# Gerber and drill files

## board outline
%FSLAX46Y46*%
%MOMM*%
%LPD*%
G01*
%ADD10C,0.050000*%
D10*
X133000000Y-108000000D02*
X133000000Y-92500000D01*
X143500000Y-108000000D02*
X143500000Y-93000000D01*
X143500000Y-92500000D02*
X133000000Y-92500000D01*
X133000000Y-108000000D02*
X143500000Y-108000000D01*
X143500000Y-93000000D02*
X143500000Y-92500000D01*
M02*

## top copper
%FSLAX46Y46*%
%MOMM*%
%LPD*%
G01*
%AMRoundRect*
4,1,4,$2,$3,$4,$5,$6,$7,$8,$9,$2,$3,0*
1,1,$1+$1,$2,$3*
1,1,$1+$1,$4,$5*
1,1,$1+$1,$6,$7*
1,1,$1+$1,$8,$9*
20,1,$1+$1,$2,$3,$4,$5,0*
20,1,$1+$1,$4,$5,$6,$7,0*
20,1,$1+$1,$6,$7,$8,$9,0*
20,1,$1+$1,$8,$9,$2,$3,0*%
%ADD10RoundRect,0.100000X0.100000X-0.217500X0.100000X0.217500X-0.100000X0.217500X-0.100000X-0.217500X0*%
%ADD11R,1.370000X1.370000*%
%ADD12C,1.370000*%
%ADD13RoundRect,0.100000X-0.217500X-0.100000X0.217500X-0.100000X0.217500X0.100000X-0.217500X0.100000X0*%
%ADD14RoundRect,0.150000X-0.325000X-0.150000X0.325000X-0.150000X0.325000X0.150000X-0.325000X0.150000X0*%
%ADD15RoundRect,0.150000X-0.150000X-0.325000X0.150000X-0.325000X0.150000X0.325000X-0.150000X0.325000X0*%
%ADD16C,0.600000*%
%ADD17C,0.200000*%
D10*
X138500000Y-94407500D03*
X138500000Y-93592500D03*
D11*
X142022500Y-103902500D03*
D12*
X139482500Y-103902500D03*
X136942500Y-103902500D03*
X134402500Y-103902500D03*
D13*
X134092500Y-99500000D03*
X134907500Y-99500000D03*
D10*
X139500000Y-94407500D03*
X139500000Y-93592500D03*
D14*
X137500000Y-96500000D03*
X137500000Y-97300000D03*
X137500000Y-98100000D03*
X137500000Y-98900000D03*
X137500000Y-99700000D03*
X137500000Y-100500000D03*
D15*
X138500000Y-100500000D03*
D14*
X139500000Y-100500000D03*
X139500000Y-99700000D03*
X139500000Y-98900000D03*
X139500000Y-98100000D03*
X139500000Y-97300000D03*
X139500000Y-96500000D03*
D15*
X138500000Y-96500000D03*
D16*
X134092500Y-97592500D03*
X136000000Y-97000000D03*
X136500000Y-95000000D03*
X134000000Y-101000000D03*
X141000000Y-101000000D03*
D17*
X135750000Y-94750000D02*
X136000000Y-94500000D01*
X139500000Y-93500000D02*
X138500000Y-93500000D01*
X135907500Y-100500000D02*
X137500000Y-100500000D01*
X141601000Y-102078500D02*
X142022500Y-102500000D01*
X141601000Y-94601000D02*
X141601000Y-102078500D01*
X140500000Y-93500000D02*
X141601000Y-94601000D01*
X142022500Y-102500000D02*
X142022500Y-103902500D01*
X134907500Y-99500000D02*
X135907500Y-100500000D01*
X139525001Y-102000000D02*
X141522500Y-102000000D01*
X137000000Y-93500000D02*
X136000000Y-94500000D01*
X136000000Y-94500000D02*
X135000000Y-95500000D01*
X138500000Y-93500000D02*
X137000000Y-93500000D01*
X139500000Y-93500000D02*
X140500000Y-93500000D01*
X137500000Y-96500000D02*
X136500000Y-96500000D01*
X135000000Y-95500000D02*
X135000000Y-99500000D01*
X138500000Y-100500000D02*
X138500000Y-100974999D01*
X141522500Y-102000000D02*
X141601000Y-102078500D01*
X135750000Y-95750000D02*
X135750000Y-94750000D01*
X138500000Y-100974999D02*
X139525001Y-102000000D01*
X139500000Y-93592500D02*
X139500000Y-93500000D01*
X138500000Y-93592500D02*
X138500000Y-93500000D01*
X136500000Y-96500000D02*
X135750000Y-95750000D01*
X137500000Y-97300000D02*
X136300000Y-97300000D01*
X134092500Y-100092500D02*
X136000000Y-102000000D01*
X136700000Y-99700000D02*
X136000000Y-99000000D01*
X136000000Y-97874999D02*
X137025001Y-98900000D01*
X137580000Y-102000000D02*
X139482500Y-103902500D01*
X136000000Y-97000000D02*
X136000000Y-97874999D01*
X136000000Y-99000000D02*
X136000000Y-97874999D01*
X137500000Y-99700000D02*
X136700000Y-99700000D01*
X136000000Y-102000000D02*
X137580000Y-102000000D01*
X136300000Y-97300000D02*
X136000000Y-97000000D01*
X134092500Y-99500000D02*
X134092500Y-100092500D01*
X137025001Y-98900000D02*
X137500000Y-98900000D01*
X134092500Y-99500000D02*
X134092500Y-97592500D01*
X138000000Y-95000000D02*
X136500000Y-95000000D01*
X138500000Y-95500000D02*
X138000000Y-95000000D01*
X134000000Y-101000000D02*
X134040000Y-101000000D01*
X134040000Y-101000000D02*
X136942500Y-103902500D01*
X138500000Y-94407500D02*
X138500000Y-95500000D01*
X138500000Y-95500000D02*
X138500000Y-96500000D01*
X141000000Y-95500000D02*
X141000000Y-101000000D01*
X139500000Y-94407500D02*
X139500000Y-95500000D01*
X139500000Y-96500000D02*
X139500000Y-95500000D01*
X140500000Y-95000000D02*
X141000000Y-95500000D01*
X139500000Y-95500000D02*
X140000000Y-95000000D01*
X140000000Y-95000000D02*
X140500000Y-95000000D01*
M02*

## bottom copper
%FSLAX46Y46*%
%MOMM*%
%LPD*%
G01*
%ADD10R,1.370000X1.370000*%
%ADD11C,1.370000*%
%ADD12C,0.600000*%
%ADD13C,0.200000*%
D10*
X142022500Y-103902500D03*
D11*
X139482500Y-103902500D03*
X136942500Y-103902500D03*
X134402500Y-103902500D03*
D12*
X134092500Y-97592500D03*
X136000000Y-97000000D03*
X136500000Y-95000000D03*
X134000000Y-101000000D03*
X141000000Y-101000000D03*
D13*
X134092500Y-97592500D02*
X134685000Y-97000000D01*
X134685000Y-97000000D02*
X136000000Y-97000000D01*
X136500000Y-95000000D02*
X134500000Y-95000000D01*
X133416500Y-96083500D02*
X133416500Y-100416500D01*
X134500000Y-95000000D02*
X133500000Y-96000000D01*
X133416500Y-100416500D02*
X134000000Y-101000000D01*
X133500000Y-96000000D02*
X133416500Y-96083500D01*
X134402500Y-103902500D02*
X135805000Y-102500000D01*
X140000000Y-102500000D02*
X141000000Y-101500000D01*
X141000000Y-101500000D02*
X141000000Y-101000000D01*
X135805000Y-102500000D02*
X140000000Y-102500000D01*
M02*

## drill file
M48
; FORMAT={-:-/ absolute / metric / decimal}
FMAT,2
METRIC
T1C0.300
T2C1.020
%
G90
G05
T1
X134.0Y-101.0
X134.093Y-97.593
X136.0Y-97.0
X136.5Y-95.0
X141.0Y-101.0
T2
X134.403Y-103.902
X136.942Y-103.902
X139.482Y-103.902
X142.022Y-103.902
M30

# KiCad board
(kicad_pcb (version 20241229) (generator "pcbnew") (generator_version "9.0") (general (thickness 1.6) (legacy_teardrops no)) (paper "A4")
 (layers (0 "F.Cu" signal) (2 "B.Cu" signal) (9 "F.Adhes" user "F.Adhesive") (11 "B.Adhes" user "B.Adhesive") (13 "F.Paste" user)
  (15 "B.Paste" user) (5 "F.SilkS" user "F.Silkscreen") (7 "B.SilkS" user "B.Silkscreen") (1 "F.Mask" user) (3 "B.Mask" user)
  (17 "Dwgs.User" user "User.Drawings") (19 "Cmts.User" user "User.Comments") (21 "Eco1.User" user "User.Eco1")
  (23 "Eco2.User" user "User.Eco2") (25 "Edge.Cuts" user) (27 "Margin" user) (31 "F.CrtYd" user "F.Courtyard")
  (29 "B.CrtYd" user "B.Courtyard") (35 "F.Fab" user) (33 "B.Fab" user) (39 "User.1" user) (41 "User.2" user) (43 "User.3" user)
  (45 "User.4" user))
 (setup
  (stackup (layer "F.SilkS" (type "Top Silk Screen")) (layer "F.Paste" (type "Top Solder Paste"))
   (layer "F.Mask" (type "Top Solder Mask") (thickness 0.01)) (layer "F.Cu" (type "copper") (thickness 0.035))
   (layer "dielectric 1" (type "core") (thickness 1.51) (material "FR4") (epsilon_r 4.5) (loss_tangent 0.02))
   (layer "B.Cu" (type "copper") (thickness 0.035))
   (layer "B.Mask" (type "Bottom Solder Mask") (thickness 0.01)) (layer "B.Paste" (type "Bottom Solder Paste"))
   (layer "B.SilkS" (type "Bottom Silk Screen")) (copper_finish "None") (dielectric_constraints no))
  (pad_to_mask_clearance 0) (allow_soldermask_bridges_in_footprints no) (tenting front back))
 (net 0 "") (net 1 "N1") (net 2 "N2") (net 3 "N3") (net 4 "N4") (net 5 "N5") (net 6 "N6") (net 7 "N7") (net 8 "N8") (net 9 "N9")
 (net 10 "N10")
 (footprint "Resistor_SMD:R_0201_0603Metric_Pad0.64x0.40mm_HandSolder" (layer "F.Cu") (at 138.5 94 90)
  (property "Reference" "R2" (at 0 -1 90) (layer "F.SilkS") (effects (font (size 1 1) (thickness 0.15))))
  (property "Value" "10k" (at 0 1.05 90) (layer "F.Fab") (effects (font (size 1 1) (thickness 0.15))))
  (pad "" smd roundrect (at -0.4325 0 90) (size 0.458 0.36) (layers "F.Paste") (roundrect_rratio 0.25))
  (pad "" smd roundrect (at 0.4325 0 90) (size 0.458 0.36) (layers "F.Paste") (roundrect_rratio 0.25))
  (pad "1" smd roundrect (at -0.4075 0 90) (size 0.635 0.4) (layers "F.Cu" "F.Mask") (roundrect_rratio 0.25) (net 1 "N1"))
  (pad "2" smd roundrect (at 0.4075 0 90) (size 0.635 0.4) (layers "F.Cu" "F.Mask") (roundrect_rratio 0.25) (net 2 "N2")))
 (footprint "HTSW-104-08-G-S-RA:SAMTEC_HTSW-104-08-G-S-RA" (layer "F.Cu") (at 138.2125 106.6725)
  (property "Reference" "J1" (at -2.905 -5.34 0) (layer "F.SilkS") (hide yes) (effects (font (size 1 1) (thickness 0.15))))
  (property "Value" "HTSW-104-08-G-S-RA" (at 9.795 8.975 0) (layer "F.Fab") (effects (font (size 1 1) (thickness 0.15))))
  (pad "01" thru_hole rect (at 3.81 -2.77) (size 1.37 1.37) (drill 1.02) (layers "*.Cu" "*.Mask") (remove_unused_layers no) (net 2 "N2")
   (solder_mask_margin 0.102))
  (pad "02" thru_hole circle (at 1.27 -2.77) (size 1.37 1.37) (drill 1.02) (layers "*.Cu" "*.Mask") (remove_unused_layers no) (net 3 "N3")
   (solder_mask_margin 0.102))
  (pad "03" thru_hole circle (at -1.27 -2.77) (size 1.37 1.37) (drill 1.02) (layers "*.Cu" "*.Mask") (remove_unused_layers no) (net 1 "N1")
   (solder_mask_margin 0.102))
  (pad "04" thru_hole circle (at -3.81 -2.77) (size 1.37 1.37) (drill 1.02) (layers "*.Cu" "*.Mask") (remove_unused_layers no) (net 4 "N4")
   (solder_mask_margin 0.102)))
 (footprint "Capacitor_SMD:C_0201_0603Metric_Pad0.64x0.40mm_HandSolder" (layer "F.Cu") (at 134.5 99.5)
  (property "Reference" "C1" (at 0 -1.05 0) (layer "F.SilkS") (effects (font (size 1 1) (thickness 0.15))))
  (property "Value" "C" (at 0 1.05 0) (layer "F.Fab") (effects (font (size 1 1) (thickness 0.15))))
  (pad "" smd roundrect (at -0.4325 0) (size 0.458 0.36) (layers "F.Paste") (roundrect_rratio 0.25))
  (pad "" smd roundrect (at 0.4325 0) (size 0.458 0.36) (layers "F.Paste") (roundrect_rratio 0.25))
  (pad "1" smd roundrect (at -0.4075 0) (size 0.635 0.4) (layers "F.Cu" "F.Mask") (roundrect_rratio 0.25) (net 3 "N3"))
  (pad "2" smd roundrect (at 0.4075 0) (size 0.635 0.4) (layers "F.Cu" "F.Mask") (roundrect_rratio 0.25) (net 2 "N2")))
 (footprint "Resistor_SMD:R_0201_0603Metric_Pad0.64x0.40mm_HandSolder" (layer "F.Cu") (at 139.5 94 90)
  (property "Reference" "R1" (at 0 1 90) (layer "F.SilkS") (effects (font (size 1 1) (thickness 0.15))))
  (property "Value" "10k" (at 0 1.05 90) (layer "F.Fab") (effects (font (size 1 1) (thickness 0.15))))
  (pad "" smd roundrect (at -0.4325 0 90) (size 0.458 0.36) (layers "F.Paste") (roundrect_rratio 0.25))
  (pad "" smd roundrect (at 0.4325 0 90) (size 0.458 0.36) (layers "F.Paste") (roundrect_rratio 0.25))
  (pad "1" smd roundrect (at -0.4075 0 90) (size 0.635 0.4) (layers "F.Cu" "F.Mask") (roundrect_rratio 0.25) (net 4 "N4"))
  (pad "2" smd roundrect (at 0.4075 0 90) (size 0.635 0.4) (layers "F.Cu" "F.Mask") (roundrect_rratio 0.25) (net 2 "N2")))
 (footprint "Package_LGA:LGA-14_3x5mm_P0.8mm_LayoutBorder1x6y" (layer "F.Cu") (at 138.5 98.5)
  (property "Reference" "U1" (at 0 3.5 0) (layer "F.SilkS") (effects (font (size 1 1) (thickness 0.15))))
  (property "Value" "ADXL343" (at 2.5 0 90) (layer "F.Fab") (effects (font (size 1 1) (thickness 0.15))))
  (pad "1" smd roundrect (at -1 -2) (size 0.95 0.6) (layers "F.Cu" "F.Mask" "F.Paste") (roundrect_rratio 0.25) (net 2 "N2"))
  (pad "2" smd roundrect (at -1 -1.2) (size 0.95 0.6) (layers "F.Cu" "F.Mask" "F.Paste") (roundrect_rratio 0.25) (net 3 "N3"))
  (pad "3" smd roundrect (at -1 -0.4) (size 0.95 0.6) (layers "F.Cu" "F.Mask" "F.Paste") (roundrect_rratio 0.25) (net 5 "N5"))
  (pad "4" smd roundrect (at -1 0.4) (size 0.95 0.6) (layers "F.Cu" "F.Mask" "F.Paste") (roundrect_rratio 0.25) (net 3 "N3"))
  (pad "5" smd roundrect (at -1 1.2) (size 0.95 0.6) (layers "F.Cu" "F.Mask" "F.Paste") (roundrect_rratio 0.25) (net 3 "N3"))
  (pad "6" smd roundrect (at -1 2) (size 0.95 0.6) (layers "F.Cu" "F.Mask" "F.Paste") (roundrect_rratio 0.25) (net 2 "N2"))
  (pad "7" smd roundrect (at 0 2) (size 0.6 0.95) (layers "F.Cu" "F.Mask" "F.Paste") (roundrect_rratio 0.25) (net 2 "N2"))
  (pad "8" smd roundrect (at 1 2) (size 0.95 0.6) (layers "F.Cu" "F.Mask" "F.Paste") (roundrect_rratio 0.25) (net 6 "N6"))
  (pad "9" smd roundrect (at 1 1.2) (size 0.95 0.6) (layers "F.Cu" "F.Mask" "F.Paste") (roundrect_rratio 0.25) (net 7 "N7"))
  (pad "10" smd roundrect (at 1 0.4) (size 0.95 0.6) (layers "F.Cu" "F.Mask" "F.Paste") (roundrect_rratio 0.25) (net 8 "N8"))
  (pad "11" smd roundrect (at 1 -0.4) (size 0.95 0.6) (layers "F.Cu" "F.Mask" "F.Paste") (roundrect_rratio 0.25) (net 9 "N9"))
  (pad "12" smd roundrect (at 1 -1.2) (size 0.95 0.6) (layers "F.Cu" "F.Mask" "F.Paste") (roundrect_rratio 0.25) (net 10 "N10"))
  (pad "13" smd roundrect (at 1 -2) (size 0.95 0.6) (layers "F.Cu" "F.Mask" "F.Paste") (roundrect_rratio 0.25) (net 4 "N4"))
  (pad "14" smd roundrect (at 0 -2) (size 0.6 0.95) (layers "F.Cu" "F.Mask" "F.Paste") (roundrect_rratio 0.25) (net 1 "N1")))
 (gr_line (start 133 108) (end 133 92.5) (stroke (width 0.05) (type default)) (layer "Edge.Cuts"))
 (gr_line (start 143.5 108) (end 143.5 93) (stroke (width 0.05) (type default)) (layer "Edge.Cuts"))
 (gr_line (start 143.5 92.5) (end 133 92.5) (stroke (width 0.05) (type default)) (layer "Edge.Cuts"))
 (gr_line (start 133 108) (end 143.5 108) (stroke (width 0.05) (type default)) (layer "Edge.Cuts"))
 (gr_line (start 143.5 93) (end 143.5 92.5) (stroke (width 0.05) (type default)) (layer "Edge.Cuts"))
 (segment (start 135.75 94.75) (end 136 94.5) (width 0.2) (layer "F.Cu") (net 2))
 (segment (start 139.5 93.5) (end 138.5 93.5) (width 0.2) (layer "F.Cu") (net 2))
 (segment (start 135.9075 100.5) (end 137.5 100.5) (width 0.2) (layer "F.Cu") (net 2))
 (segment (start 141.601 102.0785) (end 142.0225 102.5) (width 0.2) (layer "F.Cu") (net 2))
 (segment (start 141.601 94.601) (end 141.601 102.0785) (width 0.2) (layer "F.Cu") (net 2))
 (segment (start 140.5 93.5) (end 141.601 94.601) (width 0.2) (layer "F.Cu") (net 2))
 (segment (start 142.0225 102.5) (end 142.0225 103.9025) (width 0.2) (layer "F.Cu") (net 2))
 (segment (start 134.9075 99.5) (end 135.9075 100.5) (width 0.2) (layer "F.Cu") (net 2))
 (segment (start 139.525001 102) (end 141.5225 102) (width 0.2) (layer "F.Cu") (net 2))
 (segment (start 137 93.5) (end 136 94.5) (width 0.2) (layer "F.Cu") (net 2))
 (segment (start 136 94.5) (end 135 95.5) (width 0.2) (layer "F.Cu") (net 2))
 (segment (start 138.5 93.5) (end 137 93.5) (width 0.2) (layer "F.Cu") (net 2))
 (segment (start 139.5 93.5) (end 140.5 93.5) (width 0.2) (layer "F.Cu") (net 2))
 (segment (start 137.5 96.5) (end 136.5 96.5) (width 0.2) (layer "F.Cu") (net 2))
 (segment (start 135 95.5) (end 135 99.5) (width 0.2) (layer "F.Cu") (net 2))
 (segment (start 138.5 100.5) (end 138.5 100.974999) (width 0.2) (layer "F.Cu") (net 2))
 (segment (start 141.5225 102) (end 141.601 102.0785) (width 0.2) (layer "F.Cu") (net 2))
 (segment (start 135.75 95.75) (end 135.75 94.75) (width 0.2) (layer "F.Cu") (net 2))
 (segment (start 138.5 100.974999) (end 139.525001 102) (width 0.2) (layer "F.Cu") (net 2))
 (segment (start 139.5 93.5925) (end 139.5 93.5) (width 0.2) (layer "F.Cu") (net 2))
 (segment (start 138.5 93.5925) (end 138.5 93.5) (width 0.2) (layer "F.Cu") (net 2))
 (segment (start 136.5 96.5) (end 135.75 95.75) (width 0.2) (layer "F.Cu") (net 2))
 (segment (start 137.5 97.3) (end 136.3 97.3) (width 0.2) (layer "F.Cu") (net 3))
 (segment (start 134.0925 100.0925) (end 136 102) (width 0.2) (layer "F.Cu") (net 3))
 (segment (start 136.7 99.7) (end 136 99) (width 0.2) (layer "F.Cu") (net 3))
 (segment (start 136 97.874999) (end 137.025001 98.9) (width 0.2) (layer "F.Cu") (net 3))
 (segment (start 137.58 102) (end 139.4825 103.9025) (width 0.2) (layer "F.Cu") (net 3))
 (segment (start 136 97) (end 136 97.874999) (width 0.2) (layer "F.Cu") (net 3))
 (segment (start 136 99) (end 136 97.874999) (width 0.2) (layer "F.Cu") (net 3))
 (segment (start 137.5 99.7) (end 136.7 99.7) (width 0.2) (layer "F.Cu") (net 3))
 (segment (start 136 102) (end 137.58 102) (width 0.2) (layer "F.Cu") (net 3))
 (segment (start 136.3 97.3) (end 136 97) (width 0.2) (layer "F.Cu") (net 3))
 (segment (start 134.0925 99.5) (end 134.0925 100.0925) (width 0.2) (layer "F.Cu") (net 3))
 (segment (start 137.025001 98.9) (end 137.5 98.9) (width 0.2) (layer "F.Cu") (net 3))
 (segment (start 134.0925 99.5) (end 134.0925 97.5925) (width 0.2) (layer "F.Cu") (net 3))
 (via (at 134.0925 97.5925) (size 0.6) (drill 0.3) (layers "F.Cu" "B.Cu") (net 3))
 (via (at 136 97) (size 0.6) (drill 0.3) (layers "F.Cu" "B.Cu") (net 3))
 (segment (start 134.0925 97.5925) (end 134.685 97) (width 0.2) (layer "B.Cu") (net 3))
 (segment (start 134.685 97) (end 136 97) (width 0.2) (layer "B.Cu") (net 3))
 (segment (start 138 95) (end 136.5 95) (width 0.2) (layer "F.Cu") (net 1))
 (segment (start 138.5 95.5) (end 138 95) (width 0.2) (layer "F.Cu") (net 1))
 (segment (start 134 101) (end 134.04 101) (width 0.2) (layer "F.Cu") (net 1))
 (segment (start 134.04 101) (end 136.9425 103.9025) (width 0.2) (layer "F.Cu") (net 1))
 (segment (start 138.5 94.4075) (end 138.5 95.5) (width 0.2) (layer "F.Cu") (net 1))
 (segment (start 138.5 95.5) (end 138.5 96.5) (width 0.2) (layer "F.Cu") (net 1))
 (via (at 136.5 95) (size 0.6) (drill 0.3) (layers "F.Cu" "B.Cu") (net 1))
 (via (at 134 101) (size 0.6) (drill 0.3) (layers "F.Cu" "B.Cu") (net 1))
 (segment (start 136.5 95) (end 134.5 95) (width 0.2) (layer "B.Cu") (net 1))
 (segment (start 133.4165 96.0835) (end 133.4165 100.4165) (width 0.2) (layer "B.Cu") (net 1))
 (segment (start 134.5 95) (end 133.5 96) (width 0.2) (layer "B.Cu") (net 1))
 (segment (start 133.4165 100.4165) (end 134 101) (width 0.2) (layer "B.Cu") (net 1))
 (segment (start 133.5 96) (end 133.4165 96.0835) (width 0.2) (layer "B.Cu") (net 1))
 (segment (start 141 95.5) (end 141 101) (width 0.2) (layer "F.Cu") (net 4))
 (segment (start 139.5 94.4075) (end 139.5 95.5) (width 0.2) (layer "F.Cu") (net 4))
 (segment (start 139.5 96.5) (end 139.5 95.5) (width 0.2) (layer "F.Cu") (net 4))
 (segment (start 140.5 95) (end 141 95.5) (width 0.2) (layer "F.Cu") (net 4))
 (segment (start 139.5 95.5) (end 140 95) (width 0.2) (layer "F.Cu") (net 4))
 (segment (start 140 95) (end 140.5 95) (width 0.2) (layer "F.Cu") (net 4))
 (via (at 141 101) (size 0.6) (drill 0.3) (layers "F.Cu" "B.Cu") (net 4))
 (segment (start 134.4025 103.9025) (end 135.805 102.5) (width 0.2) (layer "B.Cu") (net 4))
 (segment (start 140 102.5) (end 141 101.5) (width 0.2) (layer "B.Cu") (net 4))
 (segment (start 141 101.5) (end 141 101) (width 0.2) (layer "B.Cu") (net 4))
 (segment (start 135.805 102.5) (end 140 102.5) (width 0.2) (layer "B.Cu") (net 4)))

